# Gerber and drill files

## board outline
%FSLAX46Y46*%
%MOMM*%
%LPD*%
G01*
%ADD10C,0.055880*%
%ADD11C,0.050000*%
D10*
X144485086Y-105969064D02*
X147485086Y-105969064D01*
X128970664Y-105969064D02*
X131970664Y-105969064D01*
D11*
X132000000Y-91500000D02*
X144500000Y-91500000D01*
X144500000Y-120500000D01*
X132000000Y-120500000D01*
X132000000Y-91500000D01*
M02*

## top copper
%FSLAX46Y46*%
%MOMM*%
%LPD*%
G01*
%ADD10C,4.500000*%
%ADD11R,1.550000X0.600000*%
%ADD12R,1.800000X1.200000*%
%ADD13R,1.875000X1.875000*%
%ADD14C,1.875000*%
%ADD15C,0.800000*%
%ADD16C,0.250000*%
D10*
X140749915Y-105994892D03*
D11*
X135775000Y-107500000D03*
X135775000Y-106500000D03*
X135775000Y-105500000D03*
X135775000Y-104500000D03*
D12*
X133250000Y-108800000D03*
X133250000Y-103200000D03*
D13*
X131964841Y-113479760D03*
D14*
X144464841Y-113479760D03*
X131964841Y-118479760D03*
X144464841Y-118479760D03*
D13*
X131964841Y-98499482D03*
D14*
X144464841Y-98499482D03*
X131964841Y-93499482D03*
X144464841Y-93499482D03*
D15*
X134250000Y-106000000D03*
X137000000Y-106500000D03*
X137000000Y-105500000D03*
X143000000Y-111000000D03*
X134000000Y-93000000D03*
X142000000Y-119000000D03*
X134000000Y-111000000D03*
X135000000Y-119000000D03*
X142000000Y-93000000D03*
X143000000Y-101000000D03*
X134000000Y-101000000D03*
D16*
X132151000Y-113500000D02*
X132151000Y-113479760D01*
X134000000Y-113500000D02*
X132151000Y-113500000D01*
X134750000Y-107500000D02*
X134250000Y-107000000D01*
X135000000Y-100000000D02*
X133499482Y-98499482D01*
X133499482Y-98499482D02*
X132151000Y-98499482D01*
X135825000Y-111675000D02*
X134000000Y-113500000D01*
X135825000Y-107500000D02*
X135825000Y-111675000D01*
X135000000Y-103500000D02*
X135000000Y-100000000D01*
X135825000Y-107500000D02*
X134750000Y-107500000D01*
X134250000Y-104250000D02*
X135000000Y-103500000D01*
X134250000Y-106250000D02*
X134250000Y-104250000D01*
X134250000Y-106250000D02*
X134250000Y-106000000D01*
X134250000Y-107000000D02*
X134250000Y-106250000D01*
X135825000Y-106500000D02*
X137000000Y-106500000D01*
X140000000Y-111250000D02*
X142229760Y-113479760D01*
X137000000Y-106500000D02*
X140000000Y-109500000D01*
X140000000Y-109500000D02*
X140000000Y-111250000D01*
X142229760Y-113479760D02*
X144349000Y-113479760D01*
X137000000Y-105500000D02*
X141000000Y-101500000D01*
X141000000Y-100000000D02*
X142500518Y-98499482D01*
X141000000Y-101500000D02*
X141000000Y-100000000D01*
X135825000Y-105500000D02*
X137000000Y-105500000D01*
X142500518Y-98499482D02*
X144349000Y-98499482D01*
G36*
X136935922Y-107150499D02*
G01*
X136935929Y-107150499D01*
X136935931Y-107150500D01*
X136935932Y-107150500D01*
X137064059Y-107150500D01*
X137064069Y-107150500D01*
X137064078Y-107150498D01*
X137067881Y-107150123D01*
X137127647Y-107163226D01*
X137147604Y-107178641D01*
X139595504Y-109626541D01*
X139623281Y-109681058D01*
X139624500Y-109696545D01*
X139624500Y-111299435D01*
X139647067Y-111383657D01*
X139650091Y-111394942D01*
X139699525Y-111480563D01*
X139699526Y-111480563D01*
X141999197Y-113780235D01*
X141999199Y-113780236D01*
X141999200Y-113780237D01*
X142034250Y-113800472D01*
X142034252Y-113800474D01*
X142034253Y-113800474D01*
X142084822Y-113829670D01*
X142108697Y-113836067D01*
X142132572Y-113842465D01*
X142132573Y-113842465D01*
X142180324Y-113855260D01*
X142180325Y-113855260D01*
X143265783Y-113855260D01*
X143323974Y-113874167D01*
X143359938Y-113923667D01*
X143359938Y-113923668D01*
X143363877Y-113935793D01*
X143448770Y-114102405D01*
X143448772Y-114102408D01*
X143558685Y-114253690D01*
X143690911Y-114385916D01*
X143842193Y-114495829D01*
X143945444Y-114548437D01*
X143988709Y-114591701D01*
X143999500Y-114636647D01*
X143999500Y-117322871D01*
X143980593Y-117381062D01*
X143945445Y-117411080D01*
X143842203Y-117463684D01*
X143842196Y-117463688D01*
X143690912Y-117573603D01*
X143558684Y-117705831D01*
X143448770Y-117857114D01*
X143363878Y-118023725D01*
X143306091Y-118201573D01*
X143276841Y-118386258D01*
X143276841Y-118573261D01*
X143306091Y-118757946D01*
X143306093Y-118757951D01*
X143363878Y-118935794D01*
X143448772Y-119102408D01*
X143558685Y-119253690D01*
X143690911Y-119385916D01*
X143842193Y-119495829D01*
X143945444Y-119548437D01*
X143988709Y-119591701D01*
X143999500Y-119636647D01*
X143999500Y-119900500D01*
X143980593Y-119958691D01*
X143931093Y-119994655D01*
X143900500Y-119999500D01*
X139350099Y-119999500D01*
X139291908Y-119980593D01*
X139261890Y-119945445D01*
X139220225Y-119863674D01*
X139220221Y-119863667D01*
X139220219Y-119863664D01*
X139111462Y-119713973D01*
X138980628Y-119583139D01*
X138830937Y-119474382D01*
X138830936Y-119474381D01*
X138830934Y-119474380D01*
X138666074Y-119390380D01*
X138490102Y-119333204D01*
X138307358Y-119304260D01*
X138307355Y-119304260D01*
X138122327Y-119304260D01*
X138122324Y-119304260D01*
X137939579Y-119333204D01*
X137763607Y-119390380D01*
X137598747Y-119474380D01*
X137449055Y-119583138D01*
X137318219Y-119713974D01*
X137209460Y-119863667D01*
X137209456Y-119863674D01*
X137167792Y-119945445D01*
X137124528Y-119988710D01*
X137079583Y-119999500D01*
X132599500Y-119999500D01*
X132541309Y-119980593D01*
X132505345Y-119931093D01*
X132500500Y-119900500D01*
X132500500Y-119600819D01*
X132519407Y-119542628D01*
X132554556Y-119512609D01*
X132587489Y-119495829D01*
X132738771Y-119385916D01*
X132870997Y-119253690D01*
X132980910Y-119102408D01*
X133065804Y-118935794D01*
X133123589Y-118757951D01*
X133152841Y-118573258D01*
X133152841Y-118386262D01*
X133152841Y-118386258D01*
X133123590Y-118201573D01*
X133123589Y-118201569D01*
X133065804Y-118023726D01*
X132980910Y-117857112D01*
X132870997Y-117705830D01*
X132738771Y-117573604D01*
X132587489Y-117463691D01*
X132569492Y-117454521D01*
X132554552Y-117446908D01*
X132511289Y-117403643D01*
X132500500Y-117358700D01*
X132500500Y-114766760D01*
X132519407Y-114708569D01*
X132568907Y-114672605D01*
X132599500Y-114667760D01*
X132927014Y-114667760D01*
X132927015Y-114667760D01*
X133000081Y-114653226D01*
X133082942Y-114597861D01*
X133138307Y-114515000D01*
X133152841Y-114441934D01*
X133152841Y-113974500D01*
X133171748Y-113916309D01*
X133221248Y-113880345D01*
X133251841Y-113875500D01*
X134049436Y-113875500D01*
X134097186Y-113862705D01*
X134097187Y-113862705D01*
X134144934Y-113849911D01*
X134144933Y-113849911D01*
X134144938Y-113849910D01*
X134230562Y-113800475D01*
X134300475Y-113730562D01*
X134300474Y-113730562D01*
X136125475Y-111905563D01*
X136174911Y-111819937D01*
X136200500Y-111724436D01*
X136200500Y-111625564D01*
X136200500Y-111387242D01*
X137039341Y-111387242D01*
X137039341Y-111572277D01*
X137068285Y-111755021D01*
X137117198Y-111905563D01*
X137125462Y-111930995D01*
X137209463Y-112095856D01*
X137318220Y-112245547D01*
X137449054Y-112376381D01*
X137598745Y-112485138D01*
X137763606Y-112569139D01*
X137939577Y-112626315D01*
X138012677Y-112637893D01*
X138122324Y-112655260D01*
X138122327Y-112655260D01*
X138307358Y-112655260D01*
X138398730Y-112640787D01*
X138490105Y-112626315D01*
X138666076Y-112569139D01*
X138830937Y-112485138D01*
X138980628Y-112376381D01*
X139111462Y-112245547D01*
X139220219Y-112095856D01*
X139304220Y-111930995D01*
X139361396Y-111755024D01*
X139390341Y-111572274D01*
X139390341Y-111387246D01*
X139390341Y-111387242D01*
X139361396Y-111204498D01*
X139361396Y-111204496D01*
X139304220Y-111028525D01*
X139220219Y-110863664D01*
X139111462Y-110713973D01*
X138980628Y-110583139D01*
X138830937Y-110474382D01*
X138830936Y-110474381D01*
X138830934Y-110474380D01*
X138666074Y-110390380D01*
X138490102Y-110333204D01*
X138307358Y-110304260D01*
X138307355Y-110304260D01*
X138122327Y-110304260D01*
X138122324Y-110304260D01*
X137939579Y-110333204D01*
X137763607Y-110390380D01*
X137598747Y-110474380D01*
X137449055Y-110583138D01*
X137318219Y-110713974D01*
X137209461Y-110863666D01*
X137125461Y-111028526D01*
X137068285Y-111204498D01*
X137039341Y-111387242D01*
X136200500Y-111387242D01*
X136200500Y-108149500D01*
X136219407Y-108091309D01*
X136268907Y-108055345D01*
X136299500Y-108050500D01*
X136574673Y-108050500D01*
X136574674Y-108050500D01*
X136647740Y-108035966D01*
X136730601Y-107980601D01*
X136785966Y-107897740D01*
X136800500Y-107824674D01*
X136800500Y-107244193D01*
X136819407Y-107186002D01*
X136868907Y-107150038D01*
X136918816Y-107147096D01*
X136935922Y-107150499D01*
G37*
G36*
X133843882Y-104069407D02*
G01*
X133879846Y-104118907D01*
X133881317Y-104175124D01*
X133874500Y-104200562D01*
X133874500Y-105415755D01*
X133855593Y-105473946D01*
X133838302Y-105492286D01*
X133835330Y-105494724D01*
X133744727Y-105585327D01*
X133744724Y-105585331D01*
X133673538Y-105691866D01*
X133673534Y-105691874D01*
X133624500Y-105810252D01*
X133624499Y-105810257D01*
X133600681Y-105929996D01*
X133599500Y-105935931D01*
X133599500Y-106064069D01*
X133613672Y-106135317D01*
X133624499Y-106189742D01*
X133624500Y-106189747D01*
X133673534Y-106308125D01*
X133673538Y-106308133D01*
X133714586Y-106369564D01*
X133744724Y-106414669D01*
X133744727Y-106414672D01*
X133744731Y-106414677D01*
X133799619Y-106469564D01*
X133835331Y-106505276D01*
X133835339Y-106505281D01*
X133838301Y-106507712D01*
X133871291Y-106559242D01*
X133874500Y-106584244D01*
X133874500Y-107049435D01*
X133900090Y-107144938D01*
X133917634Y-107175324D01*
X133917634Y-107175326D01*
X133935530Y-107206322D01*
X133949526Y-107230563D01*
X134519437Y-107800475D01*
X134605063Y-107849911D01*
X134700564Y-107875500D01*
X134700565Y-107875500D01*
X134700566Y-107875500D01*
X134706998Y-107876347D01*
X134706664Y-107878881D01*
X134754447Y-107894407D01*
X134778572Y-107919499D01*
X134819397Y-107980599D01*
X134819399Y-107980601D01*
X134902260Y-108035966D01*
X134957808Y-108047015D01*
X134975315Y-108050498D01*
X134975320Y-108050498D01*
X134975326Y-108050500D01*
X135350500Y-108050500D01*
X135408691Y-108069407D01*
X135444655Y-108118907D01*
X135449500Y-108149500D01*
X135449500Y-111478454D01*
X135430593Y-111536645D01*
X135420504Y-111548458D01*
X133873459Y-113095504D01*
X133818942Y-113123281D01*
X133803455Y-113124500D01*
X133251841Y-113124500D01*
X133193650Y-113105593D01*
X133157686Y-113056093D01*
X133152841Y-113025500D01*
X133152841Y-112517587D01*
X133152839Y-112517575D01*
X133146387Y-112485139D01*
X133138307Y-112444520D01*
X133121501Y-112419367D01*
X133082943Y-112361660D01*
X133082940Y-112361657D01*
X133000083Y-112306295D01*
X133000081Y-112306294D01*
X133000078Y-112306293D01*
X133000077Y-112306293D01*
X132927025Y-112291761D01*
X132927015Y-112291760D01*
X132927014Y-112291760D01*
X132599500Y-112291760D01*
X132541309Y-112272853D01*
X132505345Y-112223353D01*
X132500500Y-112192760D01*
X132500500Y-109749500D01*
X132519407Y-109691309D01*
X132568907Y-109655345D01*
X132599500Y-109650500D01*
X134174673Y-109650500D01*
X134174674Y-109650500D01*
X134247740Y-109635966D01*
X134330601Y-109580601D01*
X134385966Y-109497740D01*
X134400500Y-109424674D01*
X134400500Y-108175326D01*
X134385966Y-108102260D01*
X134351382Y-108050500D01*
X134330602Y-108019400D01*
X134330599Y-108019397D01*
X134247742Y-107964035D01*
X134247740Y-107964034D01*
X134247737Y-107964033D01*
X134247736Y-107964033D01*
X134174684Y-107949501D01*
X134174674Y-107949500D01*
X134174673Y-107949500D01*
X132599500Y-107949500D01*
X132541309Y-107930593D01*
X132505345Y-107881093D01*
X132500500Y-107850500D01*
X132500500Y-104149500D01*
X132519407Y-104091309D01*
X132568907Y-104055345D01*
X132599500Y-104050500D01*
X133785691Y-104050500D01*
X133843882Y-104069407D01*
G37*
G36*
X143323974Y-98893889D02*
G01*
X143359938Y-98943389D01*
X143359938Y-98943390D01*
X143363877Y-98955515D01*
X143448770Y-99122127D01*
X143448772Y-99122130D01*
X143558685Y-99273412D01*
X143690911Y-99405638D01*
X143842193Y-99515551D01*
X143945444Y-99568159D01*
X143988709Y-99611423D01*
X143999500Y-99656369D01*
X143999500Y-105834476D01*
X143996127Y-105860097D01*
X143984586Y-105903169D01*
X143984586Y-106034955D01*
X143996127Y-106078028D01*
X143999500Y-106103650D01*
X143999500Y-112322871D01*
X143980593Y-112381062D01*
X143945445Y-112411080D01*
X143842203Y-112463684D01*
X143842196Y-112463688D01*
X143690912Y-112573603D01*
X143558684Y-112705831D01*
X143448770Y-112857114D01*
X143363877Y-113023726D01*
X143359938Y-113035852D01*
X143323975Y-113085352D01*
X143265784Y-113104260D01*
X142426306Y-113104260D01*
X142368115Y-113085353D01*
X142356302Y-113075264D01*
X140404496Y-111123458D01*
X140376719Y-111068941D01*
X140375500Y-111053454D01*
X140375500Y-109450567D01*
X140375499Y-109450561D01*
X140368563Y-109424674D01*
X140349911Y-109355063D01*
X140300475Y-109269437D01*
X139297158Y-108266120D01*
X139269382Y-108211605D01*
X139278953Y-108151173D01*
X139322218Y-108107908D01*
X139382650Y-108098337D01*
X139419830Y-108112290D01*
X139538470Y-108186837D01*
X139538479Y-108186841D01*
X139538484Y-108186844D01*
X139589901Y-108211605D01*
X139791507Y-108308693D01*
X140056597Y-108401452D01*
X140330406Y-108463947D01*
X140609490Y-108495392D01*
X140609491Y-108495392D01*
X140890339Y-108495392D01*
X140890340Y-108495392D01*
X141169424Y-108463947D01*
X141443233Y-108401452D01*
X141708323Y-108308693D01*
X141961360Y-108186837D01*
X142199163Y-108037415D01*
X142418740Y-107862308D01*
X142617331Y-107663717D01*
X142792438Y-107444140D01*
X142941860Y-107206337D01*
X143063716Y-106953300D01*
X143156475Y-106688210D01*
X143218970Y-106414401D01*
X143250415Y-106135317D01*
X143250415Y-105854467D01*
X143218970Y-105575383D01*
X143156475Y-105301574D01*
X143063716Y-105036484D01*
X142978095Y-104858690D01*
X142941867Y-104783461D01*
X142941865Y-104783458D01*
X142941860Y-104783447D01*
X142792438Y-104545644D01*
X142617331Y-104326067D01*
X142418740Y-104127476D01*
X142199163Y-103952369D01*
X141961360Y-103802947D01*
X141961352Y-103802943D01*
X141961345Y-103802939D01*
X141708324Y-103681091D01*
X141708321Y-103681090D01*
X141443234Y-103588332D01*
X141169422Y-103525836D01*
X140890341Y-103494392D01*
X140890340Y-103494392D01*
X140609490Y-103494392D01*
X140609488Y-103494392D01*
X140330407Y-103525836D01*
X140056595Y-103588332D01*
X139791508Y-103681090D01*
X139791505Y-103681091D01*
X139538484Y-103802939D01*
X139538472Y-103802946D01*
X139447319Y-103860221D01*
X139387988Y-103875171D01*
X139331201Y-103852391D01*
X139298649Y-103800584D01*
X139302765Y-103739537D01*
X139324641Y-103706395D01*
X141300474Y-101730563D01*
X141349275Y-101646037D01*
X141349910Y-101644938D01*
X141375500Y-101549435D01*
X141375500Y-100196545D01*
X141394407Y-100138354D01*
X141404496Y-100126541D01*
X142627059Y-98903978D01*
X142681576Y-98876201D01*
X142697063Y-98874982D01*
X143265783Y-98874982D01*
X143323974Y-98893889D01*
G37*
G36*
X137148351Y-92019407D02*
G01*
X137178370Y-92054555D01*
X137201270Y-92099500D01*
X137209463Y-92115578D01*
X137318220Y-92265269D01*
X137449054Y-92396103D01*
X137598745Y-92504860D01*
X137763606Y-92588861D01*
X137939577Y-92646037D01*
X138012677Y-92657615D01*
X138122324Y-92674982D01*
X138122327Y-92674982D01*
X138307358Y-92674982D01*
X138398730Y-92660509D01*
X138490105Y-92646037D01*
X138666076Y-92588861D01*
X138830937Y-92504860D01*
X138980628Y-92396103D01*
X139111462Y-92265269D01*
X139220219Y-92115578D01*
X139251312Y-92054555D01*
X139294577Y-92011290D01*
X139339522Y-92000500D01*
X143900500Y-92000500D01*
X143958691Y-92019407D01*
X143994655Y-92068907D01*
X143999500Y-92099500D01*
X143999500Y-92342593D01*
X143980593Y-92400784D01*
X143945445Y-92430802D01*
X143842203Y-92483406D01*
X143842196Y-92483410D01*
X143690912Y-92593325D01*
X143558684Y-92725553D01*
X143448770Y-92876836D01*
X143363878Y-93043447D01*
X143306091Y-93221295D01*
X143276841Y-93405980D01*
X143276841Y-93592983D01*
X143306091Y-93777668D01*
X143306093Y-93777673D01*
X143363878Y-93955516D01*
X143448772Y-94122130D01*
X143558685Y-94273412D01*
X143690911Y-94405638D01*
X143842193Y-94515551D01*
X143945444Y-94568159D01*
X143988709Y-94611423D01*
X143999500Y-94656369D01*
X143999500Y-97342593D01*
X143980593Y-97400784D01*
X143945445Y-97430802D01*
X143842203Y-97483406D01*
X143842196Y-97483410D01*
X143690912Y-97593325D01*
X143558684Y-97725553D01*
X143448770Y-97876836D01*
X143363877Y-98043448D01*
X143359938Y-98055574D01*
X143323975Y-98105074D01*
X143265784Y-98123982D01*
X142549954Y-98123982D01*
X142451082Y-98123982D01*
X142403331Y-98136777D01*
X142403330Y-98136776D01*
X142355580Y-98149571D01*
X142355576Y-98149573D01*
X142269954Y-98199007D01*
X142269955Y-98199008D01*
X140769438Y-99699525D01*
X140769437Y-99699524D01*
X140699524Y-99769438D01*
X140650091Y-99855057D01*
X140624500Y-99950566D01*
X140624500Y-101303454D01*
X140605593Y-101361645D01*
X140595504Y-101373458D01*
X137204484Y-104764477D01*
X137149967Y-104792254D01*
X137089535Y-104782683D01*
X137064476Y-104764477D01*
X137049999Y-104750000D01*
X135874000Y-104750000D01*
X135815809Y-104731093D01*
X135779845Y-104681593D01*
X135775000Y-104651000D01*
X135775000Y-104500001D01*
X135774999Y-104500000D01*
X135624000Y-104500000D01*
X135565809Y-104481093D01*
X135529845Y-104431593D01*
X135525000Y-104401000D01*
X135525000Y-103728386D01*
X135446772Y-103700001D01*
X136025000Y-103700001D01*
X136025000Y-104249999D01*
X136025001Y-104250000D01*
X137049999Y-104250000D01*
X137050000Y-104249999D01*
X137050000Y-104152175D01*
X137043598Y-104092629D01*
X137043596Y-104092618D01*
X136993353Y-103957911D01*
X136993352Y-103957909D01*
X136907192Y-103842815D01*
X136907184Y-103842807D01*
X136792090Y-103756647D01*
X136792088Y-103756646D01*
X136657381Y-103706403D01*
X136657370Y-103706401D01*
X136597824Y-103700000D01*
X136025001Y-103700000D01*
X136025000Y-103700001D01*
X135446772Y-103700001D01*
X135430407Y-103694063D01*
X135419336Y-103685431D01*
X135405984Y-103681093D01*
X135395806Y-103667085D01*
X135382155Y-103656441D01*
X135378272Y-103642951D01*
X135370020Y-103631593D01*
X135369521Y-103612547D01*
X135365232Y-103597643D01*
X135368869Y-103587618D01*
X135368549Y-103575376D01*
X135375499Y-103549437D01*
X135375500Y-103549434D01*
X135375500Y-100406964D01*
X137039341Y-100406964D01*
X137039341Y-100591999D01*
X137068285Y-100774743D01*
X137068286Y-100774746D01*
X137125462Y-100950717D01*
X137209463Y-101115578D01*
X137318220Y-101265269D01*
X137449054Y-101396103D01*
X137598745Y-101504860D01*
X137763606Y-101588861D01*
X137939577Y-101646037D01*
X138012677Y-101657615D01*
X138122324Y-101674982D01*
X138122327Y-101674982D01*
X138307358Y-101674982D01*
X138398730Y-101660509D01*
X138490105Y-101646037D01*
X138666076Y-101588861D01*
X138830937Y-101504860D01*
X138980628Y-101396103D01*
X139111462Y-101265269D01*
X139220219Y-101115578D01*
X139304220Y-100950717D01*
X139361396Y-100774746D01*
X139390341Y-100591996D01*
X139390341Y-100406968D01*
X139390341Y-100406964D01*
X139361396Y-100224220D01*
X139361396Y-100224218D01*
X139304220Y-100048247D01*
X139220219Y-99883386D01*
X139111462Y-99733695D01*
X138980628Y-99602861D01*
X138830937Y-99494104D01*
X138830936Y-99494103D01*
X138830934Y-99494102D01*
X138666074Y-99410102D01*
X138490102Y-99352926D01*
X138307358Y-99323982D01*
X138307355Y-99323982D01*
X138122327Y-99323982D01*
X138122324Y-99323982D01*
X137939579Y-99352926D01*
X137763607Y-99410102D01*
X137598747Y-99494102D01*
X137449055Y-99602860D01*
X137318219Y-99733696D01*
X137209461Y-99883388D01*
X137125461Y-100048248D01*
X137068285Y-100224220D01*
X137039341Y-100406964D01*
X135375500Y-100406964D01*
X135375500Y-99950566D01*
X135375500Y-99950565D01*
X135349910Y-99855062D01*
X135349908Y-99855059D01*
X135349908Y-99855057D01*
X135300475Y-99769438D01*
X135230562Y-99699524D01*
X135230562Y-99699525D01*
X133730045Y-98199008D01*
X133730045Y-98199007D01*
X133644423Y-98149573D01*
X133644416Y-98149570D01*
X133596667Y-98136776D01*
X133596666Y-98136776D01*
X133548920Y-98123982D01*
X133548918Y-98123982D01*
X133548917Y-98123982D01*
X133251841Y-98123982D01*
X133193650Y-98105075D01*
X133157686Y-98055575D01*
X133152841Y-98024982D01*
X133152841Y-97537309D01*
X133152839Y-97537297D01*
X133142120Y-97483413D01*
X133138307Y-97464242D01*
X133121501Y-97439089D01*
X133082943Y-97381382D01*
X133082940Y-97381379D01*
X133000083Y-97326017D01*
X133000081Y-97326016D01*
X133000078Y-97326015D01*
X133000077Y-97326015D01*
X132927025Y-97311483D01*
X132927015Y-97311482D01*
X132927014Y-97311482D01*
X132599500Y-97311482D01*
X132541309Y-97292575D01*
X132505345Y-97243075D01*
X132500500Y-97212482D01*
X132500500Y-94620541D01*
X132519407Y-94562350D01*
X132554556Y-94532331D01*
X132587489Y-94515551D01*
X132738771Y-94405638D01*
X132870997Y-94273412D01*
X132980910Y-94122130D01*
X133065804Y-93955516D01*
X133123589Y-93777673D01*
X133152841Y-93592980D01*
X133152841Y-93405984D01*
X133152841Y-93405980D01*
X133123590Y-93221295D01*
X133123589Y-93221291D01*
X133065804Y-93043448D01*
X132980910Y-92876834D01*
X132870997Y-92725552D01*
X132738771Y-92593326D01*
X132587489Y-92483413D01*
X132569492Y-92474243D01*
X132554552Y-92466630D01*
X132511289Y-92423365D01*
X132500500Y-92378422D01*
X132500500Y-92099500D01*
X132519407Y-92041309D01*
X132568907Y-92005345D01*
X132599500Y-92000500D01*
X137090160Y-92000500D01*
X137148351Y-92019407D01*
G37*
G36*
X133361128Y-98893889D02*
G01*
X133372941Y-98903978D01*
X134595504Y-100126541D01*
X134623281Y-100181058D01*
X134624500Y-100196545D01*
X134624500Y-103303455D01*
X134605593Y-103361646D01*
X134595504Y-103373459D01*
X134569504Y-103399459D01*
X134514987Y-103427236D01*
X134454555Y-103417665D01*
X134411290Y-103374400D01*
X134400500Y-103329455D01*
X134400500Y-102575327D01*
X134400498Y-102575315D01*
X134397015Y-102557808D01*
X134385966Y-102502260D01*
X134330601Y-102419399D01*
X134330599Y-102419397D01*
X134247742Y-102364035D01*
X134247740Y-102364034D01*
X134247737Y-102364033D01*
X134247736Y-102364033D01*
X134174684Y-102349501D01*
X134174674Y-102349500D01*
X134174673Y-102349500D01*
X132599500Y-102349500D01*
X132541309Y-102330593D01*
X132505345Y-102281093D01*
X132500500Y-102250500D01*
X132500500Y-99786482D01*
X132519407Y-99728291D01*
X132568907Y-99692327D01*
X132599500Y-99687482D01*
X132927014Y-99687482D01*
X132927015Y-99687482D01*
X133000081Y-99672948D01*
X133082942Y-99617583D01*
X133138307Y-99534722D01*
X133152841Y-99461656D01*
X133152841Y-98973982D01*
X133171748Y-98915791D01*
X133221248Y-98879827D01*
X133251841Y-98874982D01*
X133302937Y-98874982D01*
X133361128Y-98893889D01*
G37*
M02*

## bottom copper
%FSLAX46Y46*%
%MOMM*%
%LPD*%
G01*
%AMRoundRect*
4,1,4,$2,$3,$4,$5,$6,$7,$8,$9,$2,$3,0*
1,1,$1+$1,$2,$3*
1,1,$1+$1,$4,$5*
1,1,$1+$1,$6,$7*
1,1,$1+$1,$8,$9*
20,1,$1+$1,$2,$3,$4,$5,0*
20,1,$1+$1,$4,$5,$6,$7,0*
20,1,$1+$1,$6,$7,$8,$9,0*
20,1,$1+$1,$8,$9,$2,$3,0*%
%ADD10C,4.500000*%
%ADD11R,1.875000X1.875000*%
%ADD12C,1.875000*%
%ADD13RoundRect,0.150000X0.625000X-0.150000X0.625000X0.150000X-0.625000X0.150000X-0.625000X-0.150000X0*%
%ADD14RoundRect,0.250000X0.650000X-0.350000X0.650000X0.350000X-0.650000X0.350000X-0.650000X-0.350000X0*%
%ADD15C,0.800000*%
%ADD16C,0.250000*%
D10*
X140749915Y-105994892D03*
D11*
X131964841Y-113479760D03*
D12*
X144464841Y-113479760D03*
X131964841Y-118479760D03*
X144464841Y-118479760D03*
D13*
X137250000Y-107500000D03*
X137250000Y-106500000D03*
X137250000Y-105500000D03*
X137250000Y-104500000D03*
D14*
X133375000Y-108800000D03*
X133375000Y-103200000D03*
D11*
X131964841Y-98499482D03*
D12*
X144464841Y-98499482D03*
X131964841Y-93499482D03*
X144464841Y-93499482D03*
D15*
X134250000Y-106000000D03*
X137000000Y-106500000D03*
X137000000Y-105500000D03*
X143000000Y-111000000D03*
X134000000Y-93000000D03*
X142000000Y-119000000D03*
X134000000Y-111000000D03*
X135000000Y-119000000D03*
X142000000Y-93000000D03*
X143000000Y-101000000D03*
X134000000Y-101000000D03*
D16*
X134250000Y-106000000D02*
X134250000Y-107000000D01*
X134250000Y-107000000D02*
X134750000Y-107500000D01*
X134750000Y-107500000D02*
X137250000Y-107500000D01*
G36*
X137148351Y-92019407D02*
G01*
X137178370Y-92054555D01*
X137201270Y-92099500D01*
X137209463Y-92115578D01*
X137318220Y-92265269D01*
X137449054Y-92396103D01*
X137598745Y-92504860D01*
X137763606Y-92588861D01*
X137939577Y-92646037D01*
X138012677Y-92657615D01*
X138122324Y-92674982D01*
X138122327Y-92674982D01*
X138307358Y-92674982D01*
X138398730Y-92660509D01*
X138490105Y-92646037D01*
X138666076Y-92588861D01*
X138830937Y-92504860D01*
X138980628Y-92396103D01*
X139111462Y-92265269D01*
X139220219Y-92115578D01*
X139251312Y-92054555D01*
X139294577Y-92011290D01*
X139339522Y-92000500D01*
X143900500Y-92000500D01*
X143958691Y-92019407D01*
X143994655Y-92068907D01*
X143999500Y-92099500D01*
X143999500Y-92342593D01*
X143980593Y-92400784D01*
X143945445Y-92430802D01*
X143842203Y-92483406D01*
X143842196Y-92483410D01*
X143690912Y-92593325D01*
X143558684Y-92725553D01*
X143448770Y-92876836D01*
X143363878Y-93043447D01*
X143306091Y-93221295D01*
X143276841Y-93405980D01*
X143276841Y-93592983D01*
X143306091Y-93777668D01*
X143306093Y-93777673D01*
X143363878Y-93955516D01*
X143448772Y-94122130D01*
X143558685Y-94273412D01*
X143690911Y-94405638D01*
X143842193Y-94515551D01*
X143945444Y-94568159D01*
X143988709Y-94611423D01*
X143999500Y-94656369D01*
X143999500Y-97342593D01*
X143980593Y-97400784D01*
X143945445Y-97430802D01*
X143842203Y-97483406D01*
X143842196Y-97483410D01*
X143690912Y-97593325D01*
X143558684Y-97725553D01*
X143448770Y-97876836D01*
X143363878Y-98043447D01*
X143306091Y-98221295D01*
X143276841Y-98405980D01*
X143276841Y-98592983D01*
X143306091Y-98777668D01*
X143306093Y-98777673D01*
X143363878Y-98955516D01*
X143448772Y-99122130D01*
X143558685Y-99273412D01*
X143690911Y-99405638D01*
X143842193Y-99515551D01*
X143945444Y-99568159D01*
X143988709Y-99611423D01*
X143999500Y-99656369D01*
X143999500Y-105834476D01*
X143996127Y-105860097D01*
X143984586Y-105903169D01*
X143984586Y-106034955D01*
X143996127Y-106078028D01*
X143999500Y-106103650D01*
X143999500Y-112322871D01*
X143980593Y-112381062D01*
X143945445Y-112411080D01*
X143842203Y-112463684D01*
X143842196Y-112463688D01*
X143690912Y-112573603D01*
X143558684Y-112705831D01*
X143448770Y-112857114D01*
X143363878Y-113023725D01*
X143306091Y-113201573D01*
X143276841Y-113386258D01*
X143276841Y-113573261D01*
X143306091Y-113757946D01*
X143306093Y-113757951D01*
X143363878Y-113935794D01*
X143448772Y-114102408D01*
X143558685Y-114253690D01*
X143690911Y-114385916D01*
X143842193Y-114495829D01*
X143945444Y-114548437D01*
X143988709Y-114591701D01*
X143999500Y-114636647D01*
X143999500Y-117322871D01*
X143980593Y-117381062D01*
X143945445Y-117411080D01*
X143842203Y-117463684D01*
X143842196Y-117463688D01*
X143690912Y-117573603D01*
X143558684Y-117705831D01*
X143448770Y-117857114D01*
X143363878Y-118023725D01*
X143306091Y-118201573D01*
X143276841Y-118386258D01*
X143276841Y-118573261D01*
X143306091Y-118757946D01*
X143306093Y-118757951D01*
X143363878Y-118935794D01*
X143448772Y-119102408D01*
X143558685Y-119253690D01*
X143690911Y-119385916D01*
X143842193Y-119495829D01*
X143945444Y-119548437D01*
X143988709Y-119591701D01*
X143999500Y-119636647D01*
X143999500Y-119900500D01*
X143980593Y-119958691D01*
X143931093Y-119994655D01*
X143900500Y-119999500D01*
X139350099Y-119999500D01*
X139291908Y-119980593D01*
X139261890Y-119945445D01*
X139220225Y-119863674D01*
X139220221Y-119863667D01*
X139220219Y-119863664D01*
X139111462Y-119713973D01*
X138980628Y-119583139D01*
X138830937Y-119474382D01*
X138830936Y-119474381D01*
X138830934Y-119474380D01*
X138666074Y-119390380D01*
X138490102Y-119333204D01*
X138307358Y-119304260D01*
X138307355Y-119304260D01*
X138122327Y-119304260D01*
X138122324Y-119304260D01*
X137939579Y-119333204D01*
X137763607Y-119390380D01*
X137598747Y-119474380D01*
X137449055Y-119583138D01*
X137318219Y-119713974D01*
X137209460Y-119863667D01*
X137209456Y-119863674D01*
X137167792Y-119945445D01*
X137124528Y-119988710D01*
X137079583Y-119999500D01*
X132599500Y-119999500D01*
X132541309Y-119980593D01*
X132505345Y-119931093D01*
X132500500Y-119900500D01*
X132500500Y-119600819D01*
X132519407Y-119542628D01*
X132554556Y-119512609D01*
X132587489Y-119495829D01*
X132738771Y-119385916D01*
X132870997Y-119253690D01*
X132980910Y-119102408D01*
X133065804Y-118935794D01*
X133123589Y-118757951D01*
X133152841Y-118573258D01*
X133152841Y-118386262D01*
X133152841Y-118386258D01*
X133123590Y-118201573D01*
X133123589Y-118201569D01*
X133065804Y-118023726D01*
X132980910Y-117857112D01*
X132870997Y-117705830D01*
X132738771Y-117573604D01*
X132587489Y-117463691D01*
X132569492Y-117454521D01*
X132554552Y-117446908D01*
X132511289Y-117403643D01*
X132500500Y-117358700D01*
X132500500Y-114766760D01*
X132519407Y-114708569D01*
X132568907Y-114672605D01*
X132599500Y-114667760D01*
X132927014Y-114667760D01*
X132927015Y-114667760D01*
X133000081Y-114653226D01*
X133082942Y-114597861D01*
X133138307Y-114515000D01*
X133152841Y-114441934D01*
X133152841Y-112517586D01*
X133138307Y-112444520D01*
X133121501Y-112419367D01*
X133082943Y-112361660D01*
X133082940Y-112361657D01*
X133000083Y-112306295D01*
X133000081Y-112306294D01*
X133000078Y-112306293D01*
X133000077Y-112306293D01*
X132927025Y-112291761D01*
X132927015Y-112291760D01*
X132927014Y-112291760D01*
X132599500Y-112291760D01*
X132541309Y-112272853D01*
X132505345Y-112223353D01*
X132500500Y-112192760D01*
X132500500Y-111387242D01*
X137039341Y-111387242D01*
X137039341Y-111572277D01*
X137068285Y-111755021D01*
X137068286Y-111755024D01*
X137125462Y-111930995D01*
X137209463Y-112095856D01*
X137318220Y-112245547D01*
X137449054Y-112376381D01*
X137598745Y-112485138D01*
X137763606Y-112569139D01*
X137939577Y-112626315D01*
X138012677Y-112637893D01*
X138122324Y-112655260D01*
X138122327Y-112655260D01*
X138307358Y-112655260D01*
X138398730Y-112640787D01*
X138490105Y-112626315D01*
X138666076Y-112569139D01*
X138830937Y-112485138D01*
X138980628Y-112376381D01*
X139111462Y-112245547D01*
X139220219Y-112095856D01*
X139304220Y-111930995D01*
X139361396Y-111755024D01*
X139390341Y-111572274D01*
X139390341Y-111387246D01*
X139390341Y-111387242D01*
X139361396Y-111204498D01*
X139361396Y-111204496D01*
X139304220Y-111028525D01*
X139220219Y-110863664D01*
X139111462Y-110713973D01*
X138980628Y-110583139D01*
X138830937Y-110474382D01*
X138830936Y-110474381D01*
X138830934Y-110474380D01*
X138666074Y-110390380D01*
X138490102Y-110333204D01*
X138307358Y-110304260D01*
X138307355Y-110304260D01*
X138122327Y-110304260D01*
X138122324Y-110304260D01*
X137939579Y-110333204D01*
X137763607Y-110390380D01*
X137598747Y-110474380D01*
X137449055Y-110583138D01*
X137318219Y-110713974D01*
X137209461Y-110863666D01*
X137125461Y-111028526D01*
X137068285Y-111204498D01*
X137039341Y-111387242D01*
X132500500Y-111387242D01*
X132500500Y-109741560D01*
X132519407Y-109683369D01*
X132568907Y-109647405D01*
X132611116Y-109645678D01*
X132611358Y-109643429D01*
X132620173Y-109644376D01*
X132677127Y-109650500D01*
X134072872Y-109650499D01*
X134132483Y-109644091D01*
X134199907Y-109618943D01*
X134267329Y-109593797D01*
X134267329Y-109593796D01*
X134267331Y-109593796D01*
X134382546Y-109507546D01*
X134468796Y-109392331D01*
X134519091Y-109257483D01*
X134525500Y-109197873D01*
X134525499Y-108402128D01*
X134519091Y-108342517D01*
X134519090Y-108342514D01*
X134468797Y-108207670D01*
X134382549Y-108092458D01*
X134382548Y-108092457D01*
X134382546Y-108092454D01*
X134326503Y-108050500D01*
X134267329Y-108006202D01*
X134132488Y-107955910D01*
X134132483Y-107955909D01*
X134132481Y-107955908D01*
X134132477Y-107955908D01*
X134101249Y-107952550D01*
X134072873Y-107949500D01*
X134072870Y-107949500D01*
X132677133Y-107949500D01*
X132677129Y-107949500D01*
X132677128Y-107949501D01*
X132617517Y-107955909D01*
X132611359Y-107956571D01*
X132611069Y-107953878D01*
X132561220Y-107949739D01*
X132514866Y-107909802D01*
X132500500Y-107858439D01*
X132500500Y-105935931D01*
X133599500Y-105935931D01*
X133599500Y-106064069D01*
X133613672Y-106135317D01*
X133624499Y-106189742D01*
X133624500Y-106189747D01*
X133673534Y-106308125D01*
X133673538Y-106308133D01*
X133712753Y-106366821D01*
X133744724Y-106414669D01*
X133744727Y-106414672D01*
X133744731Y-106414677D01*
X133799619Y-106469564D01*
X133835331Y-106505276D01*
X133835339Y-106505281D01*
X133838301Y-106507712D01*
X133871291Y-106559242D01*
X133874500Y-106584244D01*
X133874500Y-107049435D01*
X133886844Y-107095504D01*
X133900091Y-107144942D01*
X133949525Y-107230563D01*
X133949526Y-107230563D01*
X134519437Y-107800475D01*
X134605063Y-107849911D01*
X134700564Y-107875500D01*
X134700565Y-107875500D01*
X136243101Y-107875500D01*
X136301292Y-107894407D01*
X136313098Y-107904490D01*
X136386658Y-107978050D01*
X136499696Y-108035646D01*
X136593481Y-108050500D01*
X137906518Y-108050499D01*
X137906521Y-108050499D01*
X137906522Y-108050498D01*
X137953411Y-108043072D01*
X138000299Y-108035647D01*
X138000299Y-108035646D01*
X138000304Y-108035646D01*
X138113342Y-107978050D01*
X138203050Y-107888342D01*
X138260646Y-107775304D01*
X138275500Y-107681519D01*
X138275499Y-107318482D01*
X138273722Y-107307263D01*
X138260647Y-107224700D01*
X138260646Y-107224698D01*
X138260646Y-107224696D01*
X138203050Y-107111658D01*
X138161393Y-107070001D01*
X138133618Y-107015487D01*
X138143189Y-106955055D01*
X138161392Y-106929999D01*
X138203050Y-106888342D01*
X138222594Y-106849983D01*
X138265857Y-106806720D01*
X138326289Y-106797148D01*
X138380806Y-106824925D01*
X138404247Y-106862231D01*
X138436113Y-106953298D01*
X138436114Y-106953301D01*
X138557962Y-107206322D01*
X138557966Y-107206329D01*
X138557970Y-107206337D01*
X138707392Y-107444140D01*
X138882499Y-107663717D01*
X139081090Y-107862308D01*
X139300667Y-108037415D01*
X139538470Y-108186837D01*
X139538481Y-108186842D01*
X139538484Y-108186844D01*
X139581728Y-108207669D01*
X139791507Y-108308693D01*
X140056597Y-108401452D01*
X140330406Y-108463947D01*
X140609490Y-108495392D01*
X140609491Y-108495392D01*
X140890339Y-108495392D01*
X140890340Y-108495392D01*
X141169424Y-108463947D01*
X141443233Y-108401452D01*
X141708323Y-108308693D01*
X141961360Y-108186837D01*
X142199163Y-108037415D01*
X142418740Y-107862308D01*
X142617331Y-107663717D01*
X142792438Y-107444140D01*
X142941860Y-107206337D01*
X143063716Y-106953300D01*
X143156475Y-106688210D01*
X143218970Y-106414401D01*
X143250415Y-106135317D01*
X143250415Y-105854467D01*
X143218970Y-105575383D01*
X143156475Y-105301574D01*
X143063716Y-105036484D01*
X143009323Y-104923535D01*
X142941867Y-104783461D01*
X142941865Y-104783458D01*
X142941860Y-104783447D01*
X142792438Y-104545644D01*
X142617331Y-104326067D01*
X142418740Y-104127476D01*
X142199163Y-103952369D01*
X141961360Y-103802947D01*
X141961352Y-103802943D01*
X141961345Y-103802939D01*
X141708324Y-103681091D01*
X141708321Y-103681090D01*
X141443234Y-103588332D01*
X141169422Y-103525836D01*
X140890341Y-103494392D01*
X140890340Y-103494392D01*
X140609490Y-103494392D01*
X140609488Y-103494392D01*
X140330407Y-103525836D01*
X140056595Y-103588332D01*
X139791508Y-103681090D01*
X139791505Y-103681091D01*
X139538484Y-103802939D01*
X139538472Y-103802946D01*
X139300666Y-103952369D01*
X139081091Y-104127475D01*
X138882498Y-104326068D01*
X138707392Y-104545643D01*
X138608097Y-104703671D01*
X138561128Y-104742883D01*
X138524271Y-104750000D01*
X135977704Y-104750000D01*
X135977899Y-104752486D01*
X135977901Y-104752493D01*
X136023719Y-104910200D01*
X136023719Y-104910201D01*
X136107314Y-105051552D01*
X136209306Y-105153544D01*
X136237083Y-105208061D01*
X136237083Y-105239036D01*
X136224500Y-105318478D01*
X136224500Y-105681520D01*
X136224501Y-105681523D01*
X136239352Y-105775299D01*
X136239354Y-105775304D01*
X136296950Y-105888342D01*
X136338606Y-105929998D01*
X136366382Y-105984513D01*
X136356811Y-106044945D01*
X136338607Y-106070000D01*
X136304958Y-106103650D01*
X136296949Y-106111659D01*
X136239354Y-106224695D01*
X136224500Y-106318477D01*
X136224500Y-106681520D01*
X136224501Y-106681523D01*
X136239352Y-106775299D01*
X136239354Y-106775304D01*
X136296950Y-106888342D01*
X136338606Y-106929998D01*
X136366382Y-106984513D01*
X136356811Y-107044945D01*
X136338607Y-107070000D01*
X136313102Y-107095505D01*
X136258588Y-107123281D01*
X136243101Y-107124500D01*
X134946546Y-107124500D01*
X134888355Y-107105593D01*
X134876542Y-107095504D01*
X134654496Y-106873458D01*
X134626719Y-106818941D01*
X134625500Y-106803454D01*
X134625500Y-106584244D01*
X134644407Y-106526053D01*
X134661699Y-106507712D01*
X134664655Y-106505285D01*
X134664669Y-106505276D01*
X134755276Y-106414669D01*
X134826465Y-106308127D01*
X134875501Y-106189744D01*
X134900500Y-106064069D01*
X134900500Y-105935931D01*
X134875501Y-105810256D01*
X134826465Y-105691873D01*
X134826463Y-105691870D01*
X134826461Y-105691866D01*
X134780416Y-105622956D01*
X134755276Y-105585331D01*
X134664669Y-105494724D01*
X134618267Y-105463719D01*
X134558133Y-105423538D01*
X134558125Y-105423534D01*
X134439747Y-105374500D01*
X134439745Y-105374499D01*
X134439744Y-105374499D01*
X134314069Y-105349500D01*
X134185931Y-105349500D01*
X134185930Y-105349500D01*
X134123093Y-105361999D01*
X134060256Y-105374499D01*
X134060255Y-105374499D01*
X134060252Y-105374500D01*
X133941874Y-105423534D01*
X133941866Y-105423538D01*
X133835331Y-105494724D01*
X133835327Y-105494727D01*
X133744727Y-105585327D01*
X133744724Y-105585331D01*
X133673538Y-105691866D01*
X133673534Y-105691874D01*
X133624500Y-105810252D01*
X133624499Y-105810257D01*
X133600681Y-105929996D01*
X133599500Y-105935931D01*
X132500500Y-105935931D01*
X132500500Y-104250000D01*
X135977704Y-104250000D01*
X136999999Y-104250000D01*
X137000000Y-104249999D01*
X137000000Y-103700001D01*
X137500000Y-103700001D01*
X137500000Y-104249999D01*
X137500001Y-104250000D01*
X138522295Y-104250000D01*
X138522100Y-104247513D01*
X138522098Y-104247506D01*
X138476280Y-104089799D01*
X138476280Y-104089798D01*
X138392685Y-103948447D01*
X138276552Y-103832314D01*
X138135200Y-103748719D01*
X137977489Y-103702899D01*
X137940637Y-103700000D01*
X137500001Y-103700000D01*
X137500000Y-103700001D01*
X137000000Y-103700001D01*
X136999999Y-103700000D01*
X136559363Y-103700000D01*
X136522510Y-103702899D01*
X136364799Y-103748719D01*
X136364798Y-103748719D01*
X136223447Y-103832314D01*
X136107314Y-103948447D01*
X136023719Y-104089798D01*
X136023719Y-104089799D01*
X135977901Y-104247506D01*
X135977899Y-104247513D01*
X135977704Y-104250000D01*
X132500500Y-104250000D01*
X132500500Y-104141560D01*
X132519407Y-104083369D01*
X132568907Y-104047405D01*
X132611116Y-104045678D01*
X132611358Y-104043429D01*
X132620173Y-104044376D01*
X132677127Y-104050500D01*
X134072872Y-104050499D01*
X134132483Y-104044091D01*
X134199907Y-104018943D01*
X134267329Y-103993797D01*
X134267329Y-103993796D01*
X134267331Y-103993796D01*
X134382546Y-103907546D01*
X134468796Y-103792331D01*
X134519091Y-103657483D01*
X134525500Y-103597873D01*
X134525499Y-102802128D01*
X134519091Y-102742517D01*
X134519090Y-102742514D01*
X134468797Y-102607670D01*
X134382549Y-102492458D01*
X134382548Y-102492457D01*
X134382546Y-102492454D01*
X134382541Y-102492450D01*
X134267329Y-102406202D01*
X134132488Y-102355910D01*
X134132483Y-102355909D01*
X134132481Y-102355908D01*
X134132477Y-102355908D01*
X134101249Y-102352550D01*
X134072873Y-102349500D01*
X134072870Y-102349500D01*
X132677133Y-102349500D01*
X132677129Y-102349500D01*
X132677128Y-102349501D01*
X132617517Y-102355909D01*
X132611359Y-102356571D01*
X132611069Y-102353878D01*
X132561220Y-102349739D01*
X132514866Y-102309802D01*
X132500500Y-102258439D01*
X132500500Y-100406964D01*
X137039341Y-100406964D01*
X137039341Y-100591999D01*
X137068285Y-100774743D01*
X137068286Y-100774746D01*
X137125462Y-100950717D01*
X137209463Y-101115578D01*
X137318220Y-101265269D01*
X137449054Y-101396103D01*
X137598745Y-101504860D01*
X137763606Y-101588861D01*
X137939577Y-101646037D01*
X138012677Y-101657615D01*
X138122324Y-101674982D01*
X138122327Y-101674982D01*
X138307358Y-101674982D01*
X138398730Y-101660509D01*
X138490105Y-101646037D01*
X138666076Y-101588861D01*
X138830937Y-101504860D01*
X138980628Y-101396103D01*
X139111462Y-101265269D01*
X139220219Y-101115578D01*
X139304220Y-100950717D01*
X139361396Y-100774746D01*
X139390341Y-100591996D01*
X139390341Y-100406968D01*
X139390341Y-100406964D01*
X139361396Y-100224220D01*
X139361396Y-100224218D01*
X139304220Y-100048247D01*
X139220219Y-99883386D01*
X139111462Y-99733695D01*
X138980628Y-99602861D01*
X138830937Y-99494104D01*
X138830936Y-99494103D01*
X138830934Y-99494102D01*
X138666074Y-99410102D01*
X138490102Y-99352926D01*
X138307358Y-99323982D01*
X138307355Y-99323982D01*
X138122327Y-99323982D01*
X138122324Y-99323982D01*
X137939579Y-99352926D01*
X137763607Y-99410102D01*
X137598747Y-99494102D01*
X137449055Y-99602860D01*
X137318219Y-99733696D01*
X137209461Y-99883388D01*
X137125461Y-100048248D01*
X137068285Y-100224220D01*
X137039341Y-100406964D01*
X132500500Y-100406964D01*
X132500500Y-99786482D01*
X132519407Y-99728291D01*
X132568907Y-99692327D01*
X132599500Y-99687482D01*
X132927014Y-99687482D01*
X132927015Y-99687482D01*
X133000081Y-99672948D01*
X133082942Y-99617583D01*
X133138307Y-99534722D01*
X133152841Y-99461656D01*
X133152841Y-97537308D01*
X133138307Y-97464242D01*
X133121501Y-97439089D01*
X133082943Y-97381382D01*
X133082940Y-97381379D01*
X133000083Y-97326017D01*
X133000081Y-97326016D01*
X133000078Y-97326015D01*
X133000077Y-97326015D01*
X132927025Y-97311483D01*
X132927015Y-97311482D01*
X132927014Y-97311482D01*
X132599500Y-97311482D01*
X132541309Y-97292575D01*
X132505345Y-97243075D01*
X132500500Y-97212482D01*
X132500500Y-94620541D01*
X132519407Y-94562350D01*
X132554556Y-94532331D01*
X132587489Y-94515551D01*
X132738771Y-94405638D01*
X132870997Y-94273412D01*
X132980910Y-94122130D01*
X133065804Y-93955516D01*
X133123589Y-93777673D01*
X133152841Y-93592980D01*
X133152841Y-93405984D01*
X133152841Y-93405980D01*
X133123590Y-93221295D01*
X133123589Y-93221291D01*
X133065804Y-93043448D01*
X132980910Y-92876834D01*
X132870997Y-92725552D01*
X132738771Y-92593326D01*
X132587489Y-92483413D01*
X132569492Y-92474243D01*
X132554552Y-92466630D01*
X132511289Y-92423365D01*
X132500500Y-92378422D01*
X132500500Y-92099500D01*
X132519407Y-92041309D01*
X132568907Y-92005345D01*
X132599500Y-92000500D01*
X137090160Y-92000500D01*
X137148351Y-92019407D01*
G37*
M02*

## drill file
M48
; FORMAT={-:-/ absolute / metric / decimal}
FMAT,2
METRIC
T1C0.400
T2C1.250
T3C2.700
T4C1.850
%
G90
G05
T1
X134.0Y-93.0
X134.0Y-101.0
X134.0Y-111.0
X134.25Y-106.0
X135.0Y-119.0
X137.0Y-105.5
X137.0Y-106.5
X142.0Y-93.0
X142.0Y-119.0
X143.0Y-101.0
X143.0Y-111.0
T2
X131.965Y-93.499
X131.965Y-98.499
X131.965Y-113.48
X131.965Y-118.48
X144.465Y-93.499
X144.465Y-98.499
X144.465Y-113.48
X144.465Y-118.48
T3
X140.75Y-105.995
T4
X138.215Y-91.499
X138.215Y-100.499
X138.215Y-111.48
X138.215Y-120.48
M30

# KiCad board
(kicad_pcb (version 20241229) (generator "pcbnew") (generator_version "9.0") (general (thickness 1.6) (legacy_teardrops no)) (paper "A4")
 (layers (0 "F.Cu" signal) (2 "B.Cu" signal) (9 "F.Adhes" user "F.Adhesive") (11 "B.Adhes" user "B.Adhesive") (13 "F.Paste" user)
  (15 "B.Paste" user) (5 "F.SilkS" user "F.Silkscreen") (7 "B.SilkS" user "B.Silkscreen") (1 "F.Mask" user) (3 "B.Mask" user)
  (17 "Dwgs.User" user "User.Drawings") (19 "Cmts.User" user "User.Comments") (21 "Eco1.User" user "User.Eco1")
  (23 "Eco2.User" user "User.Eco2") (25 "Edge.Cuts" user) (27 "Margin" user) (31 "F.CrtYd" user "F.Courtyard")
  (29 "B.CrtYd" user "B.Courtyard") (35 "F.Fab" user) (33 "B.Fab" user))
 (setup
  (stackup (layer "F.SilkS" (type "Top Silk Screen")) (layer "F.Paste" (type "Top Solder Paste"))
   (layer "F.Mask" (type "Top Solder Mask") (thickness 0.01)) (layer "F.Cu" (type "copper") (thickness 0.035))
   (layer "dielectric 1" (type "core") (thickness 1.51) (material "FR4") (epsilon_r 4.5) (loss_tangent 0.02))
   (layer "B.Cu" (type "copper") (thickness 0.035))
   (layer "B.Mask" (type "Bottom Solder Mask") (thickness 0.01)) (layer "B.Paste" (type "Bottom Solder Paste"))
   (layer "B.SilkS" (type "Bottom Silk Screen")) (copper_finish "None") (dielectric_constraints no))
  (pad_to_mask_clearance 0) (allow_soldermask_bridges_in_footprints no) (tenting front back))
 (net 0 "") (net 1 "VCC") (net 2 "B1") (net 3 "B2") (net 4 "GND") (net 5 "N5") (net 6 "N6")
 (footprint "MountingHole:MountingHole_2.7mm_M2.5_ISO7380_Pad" (layer "F.Cu") (at 140.749915 105.994892)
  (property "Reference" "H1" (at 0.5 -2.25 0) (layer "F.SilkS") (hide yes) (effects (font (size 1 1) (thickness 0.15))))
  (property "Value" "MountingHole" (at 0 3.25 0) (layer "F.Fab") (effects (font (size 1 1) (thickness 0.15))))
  (pad "1" thru_hole circle (at 0 0) (size 4.5 4.5) (drill 2.7) (layers "*.Cu" "*.Mask") (remove_unused_layers no)))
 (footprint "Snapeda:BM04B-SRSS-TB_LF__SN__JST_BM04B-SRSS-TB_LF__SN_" (layer "F.Cu") (at 133.25 106 90)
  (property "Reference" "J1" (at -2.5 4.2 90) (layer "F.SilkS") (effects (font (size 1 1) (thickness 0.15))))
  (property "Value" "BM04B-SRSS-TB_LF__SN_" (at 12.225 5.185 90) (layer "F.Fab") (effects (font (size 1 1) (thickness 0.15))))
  (pad "1" smd rect (at -1.5 2.525 90) (size 0.6 1.55) (layers "F.Cu" "F.Mask" "F.Paste") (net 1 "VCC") (solder_mask_margin 0.102))
  (pad "2" smd rect (at -0.5 2.525 90) (size 0.6 1.55) (layers "F.Cu" "F.Mask" "F.Paste") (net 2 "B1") (solder_mask_margin 0.102))
  (pad "3" smd rect (at 0.5 2.525 90) (size 0.6 1.55) (layers "F.Cu" "F.Mask" "F.Paste") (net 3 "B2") (solder_mask_margin 0.102))
  (pad "4" smd rect (at 1.5 2.525 90) (size 0.6 1.55) (layers "F.Cu" "F.Mask" "F.Paste") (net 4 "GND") (solder_mask_margin 0.102))
  (pad "S1" smd rect (at -2.8 0 90) (size 1.2 1.8) (layers "F.Cu" "F.Mask" "F.Paste") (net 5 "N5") (solder_mask_margin 0.102))
  (pad "S2" smd rect (at 2.8 0 90) (size 1.2 1.8) (layers "F.Cu" "F.Mask" "F.Paste") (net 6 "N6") (solder_mask_margin 0.102)))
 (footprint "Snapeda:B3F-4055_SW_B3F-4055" (layer "F.Cu") (at 138.214841 115.97976)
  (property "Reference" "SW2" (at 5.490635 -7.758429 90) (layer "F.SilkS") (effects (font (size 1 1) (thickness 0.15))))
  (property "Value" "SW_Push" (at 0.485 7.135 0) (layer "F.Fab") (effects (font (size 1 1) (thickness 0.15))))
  (pad "" np_thru_hole circle (at 0 -4.5) (size 1.85 1.85) (drill 1.85) (layers "*.Cu" "*.Mask"))
  (pad "" np_thru_hole circle (at 0 4.5) (size 1.85 1.85) (drill 1.85) (layers "*.Cu" "*.Mask"))
  (pad "1" thru_hole rect (at -6.25 -2.5) (size 1.875 1.875) (drill 1.25) (layers "*.Cu" "*.Mask") (remove_unused_layers no) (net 1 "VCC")
   (solder_mask_margin 0.102))
  (pad "2" thru_hole circle (at 6.25 -2.5) (size 1.875 1.875) (drill 1.25) (layers "*.Cu" "*.Mask") (remove_unused_layers no) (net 2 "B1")
   (solder_mask_margin 0.102))
  (pad "3" thru_hole circle (at -6.25 2.5) (size 1.875 1.875) (drill 1.25) (layers "*.Cu" "*.Mask") (remove_unused_layers no)
   (solder_mask_margin 0.102))
  (pad "4" thru_hole circle (at 6.25 2.5) (size 1.875 1.875) (drill 1.25) (layers "*.Cu" "*.Mask") (remove_unused_layers no)
   (solder_mask_margin 0.102)))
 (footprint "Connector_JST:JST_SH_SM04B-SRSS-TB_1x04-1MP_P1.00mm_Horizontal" (layer "B.Cu") (at 135.25 106 90)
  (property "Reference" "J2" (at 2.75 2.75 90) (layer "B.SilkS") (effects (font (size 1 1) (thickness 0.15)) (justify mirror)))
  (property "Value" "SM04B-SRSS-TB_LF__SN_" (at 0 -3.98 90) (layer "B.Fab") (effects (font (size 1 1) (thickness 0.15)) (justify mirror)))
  (pad "1" smd roundrect (at -1.5 2 90) (size 0.6 1.55) (layers "B.Cu" "B.Mask" "B.Paste") (roundrect_rratio 0.25) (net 1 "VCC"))
  (pad "2" smd roundrect (at -0.5 2 90) (size 0.6 1.55) (layers "B.Cu" "B.Mask" "B.Paste") (roundrect_rratio 0.25) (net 2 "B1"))
  (pad "3" smd roundrect (at 0.5 2 90) (size 0.6 1.55) (layers "B.Cu" "B.Mask" "B.Paste") (roundrect_rratio 0.25) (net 3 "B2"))
  (pad "4" smd roundrect (at 1.5 2 90) (size 0.6 1.55) (layers "B.Cu" "B.Mask" "B.Paste") (roundrect_rratio 0.25) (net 4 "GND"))
  (pad "MP" smd roundrect (at -2.8 -1.875 90) (size 1.2 1.8) (layers "B.Cu" "B.Mask" "B.Paste") (roundrect_rratio 0.208333))
  (pad "MP" smd roundrect (at 2.8 -1.875 90) (size 1.2 1.8) (layers "B.Cu" "B.Mask" "B.Paste") (roundrect_rratio 0.208333)))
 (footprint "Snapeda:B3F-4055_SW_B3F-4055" (layer "B.Cu") (at 138.214841 95.999482)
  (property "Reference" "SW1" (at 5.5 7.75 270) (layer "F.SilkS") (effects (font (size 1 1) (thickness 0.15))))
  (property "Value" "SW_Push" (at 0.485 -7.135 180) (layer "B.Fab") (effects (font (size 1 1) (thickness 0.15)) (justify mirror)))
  (pad "" np_thru_hole circle (at 0 -4.5) (size 1.85 1.85) (drill 1.85) (layers "*.Cu" "*.Mask"))
  (pad "" np_thru_hole circle (at 0 4.5) (size 1.85 1.85) (drill 1.85) (layers "*.Cu" "*.Mask"))
  (pad "1" thru_hole rect (at -6.25 2.5) (size 1.875 1.875) (drill 1.25) (layers "*.Cu" "*.Mask") (remove_unused_layers no) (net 1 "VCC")
   (solder_mask_margin 0.102))
  (pad "2" thru_hole circle (at 6.25 2.5) (size 1.875 1.875) (drill 1.25) (layers "*.Cu" "*.Mask") (remove_unused_layers no) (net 3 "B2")
   (solder_mask_margin 0.102))
  (pad "3" thru_hole circle (at -6.25 -2.5) (size 1.875 1.875) (drill 1.25) (layers "*.Cu" "*.Mask") (remove_unused_layers no)
   (solder_mask_margin 0.102))
  (pad "4" thru_hole circle (at 6.25 -2.5) (size 1.875 1.875) (drill 1.25) (layers "*.Cu" "*.Mask") (remove_unused_layers no)
   (solder_mask_margin 0.102)))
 (gr_line (start 144.485086 105.969064) (end 147.485086 105.969064) (stroke (width 0.05588) (type solid)) (layer "Edge.Cuts"))
 (gr_line (start 128.970664 105.969064) (end 131.970664 105.969064) (stroke (width 0.05588) (type solid)) (layer "Edge.Cuts"))
 (gr_rect (start 132 91.5) (end 144.5 120.5) (stroke (width 0.05) (type solid)) (fill no) (layer "Edge.Cuts"))
 (segment (start 132.151 113.5) (end 132.151 113.47976) (width 0.25) (layer "F.Cu") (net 1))
 (segment (start 134 113.5) (end 132.151 113.5) (width 0.25) (layer "F.Cu") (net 1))
 (segment (start 134.75 107.5) (end 134.25 107) (width 0.25) (layer "F.Cu") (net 1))
 (segment (start 135 100) (end 133.499482 98.499482) (width 0.25) (layer "F.Cu") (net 1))
 (segment (start 133.499482 98.499482) (end 132.151 98.499482) (width 0.25) (layer "F.Cu") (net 1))
 (segment (start 135.825 111.675) (end 134 113.5) (width 0.25) (layer "F.Cu") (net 1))
 (segment (start 135.825 107.5) (end 135.825 111.675) (width 0.25) (layer "F.Cu") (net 1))
 (segment (start 135 103.5) (end 135 100) (width 0.25) (layer "F.Cu") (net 1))
 (segment (start 135.825 107.5) (end 134.75 107.5) (width 0.25) (layer "F.Cu") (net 1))
 (segment (start 134.25 104.25) (end 135 103.5) (width 0.25) (layer "F.Cu") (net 1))
 (segment (start 134.25 106.25) (end 134.25 104.25) (width 0.25) (layer "F.Cu") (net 1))
 (segment (start 134.25 106.25) (end 134.25 106) (width 0.25) (layer "F.Cu") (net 1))
 (segment (start 134.25 107) (end 134.25 106.25) (width 0.25) (layer "F.Cu") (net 1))
 (via (at 134.25 106) (size 0.8) (drill 0.4) (layers "F.Cu" "B.Cu") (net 1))
 (segment (start 134.25 106) (end 134.25 107) (width 0.25) (layer "B.Cu") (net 1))
 (segment (start 134.25 107) (end 134.75 107.5) (width 0.25) (layer "B.Cu") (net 1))
 (segment (start 134.75 107.5) (end 137.25 107.5) (width 0.25) (layer "B.Cu") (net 1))
 (segment (start 135.825 106.5) (end 137 106.5) (width 0.25) (layer "F.Cu") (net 2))
 (segment (start 140 111.25) (end 142.22976 113.47976) (width 0.25) (layer "F.Cu") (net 2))
 (segment (start 137 106.5) (end 140 109.5) (width 0.25) (layer "F.Cu") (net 2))
 (segment (start 140 109.5) (end 140 111.25) (width 0.25) (layer "F.Cu") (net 2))
 (segment (start 142.22976 113.47976) (end 144.349 113.47976) (width 0.25) (layer "F.Cu") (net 2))
 (via (at 137 106.5) (size 0.8) (drill 0.4) (layers "F.Cu" "B.Cu") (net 2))
 (segment (start 137 105.5) (end 141 101.5) (width 0.25) (layer "F.Cu") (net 3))
 (segment (start 141 100) (end 142.500518 98.499482) (width 0.25) (layer "F.Cu") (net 3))
 (segment (start 141 101.5) (end 141 100) (width 0.25) (layer "F.Cu") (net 3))
 (segment (start 135.825 105.5) (end 137 105.5) (width 0.25) (layer "F.Cu") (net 3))
 (segment (start 142.500518 98.499482) (end 144.349 98.499482) (width 0.25) (layer "F.Cu") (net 3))
 (via (at 137 105.5) (size 0.8) (drill 0.4) (layers "F.Cu" "B.Cu") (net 3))
 (via (at 143 111) (size 0.8) (drill 0.4) (layers "F.Cu" "B.Cu") (free yes) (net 4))
 (via (at 134 93) (size 0.8) (drill 0.4) (layers "F.Cu" "B.Cu") (free yes) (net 4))
 (via (at 142 119) (size 0.8) (drill 0.4) (layers "F.Cu" "B.Cu") (free yes) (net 4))
 (via (at 134 111) (size 0.8) (drill 0.4) (layers "F.Cu" "B.Cu") (free yes) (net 4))
 (via (at 135 119) (size 0.8) (drill 0.4) (layers "F.Cu" "B.Cu") (free yes) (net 4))
 (via (at 142 93) (size 0.8) (drill 0.4) (layers "F.Cu" "B.Cu") (free yes) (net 4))
 (via (at 143 101) (size 0.8) (drill 0.4) (layers "F.Cu" "B.Cu") (free yes) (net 4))
 (via (at 134 101) (size 0.8) (drill 0.4) (layers "F.Cu" "B.Cu") (free yes) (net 4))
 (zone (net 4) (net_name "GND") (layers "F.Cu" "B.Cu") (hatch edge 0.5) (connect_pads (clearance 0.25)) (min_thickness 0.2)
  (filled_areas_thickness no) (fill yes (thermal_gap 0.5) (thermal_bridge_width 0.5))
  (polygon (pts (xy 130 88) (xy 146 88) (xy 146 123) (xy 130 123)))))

